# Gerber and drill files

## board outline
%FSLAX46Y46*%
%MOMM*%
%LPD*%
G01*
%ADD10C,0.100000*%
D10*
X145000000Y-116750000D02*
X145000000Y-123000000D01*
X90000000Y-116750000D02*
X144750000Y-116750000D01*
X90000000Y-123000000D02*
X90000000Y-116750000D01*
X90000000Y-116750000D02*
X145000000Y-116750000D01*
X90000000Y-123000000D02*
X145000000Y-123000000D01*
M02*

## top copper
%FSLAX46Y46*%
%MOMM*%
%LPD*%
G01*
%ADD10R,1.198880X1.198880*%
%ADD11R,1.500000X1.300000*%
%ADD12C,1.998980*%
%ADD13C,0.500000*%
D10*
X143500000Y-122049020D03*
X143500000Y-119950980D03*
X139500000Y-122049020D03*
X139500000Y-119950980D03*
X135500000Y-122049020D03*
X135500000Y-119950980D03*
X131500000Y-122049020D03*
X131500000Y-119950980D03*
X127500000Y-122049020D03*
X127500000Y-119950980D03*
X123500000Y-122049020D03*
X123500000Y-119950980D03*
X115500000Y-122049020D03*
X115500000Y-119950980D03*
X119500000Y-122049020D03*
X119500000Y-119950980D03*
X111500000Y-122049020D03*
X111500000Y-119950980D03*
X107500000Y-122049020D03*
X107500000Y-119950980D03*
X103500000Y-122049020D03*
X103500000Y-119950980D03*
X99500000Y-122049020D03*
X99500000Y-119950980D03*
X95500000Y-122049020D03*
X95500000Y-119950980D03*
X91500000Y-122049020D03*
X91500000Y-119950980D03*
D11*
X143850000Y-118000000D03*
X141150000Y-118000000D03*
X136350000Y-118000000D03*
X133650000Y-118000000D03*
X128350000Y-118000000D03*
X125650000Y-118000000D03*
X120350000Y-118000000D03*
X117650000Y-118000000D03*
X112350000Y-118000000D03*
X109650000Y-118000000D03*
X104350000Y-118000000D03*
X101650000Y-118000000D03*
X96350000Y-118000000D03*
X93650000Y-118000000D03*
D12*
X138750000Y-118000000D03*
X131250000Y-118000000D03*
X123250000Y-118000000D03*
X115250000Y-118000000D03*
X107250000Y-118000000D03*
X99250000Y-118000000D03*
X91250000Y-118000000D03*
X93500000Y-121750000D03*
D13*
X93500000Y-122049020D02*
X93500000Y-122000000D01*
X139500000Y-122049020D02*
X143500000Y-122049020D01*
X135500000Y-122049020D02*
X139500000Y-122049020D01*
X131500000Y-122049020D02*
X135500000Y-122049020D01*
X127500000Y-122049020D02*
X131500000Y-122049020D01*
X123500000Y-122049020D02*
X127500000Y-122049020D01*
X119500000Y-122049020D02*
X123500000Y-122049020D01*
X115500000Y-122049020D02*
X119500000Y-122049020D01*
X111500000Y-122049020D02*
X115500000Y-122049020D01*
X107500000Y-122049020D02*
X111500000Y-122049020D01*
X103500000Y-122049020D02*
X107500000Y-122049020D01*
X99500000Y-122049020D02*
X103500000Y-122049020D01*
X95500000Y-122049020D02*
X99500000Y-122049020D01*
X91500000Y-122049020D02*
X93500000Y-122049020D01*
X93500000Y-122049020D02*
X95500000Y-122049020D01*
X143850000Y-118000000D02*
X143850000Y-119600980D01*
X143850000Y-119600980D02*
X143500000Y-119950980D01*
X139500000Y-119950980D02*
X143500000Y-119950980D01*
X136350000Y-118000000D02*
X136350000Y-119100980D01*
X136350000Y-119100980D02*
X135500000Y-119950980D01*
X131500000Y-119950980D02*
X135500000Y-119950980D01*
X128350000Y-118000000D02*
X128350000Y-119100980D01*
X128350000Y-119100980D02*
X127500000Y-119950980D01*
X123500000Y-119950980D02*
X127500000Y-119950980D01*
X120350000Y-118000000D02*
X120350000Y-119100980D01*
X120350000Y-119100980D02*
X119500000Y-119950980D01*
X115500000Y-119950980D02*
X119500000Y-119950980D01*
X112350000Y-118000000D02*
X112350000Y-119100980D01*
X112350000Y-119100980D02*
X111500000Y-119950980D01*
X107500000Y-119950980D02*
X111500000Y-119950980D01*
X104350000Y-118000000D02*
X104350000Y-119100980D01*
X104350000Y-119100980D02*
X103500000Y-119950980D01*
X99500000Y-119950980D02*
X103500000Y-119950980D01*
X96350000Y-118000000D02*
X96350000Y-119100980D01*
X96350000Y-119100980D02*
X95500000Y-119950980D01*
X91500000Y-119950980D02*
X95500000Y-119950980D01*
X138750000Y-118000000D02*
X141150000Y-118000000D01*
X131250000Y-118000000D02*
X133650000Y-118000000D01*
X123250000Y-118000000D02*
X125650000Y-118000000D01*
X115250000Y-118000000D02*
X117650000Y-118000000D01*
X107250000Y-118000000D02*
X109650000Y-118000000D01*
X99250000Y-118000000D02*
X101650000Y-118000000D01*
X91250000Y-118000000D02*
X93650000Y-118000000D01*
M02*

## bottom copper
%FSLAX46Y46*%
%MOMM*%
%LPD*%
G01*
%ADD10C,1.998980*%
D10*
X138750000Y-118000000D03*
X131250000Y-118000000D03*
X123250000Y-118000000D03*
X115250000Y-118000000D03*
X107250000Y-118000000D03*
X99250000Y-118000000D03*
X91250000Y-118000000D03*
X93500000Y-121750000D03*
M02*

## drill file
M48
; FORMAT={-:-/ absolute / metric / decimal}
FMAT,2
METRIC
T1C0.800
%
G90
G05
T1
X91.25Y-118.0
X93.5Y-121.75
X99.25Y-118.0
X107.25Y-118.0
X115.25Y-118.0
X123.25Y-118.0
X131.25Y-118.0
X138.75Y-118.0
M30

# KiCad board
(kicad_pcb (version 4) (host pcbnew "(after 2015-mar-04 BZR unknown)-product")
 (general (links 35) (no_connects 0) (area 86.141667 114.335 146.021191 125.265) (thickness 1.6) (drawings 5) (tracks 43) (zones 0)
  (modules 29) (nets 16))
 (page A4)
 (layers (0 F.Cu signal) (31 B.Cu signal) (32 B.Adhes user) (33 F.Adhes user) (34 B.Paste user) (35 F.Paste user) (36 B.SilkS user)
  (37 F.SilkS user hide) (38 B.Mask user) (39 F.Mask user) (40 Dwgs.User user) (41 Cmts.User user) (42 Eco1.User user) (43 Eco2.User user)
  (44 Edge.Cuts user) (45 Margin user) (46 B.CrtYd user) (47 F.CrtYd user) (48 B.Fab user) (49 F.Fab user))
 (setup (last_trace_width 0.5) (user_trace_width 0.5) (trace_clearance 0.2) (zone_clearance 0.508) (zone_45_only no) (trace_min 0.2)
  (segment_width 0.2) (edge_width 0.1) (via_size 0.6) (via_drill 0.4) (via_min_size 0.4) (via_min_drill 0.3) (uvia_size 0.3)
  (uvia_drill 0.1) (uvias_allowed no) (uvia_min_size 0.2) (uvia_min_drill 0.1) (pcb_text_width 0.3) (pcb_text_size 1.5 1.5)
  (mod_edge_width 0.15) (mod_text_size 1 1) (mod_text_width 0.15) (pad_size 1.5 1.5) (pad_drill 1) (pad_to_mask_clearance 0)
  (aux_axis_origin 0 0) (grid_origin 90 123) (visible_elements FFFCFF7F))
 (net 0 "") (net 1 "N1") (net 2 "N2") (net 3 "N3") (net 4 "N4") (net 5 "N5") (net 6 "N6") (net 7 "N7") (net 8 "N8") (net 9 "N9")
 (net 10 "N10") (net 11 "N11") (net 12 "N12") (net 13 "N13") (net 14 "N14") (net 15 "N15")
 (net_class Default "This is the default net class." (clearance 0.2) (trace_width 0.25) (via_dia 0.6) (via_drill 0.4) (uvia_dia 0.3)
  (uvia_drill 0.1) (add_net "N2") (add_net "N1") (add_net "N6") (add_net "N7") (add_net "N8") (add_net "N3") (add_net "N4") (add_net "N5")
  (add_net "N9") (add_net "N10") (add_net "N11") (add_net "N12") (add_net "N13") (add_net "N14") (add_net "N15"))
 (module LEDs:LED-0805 (layer F.Cu) (at 143.5 121 270)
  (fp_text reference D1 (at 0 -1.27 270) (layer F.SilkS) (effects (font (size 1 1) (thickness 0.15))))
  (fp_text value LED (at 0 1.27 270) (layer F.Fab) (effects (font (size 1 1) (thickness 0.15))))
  (pad 2 smd rect (at 1.04902 0 90) (size 1.19888 1.19888) (layers F.Cu F.Paste F.Mask) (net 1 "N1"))
  (pad 1 smd rect (at -1.04902 0 90) (size 1.19888 1.19888) (layers F.Cu F.Paste F.Mask) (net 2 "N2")))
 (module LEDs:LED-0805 (layer F.Cu) (at 139.5 121 270)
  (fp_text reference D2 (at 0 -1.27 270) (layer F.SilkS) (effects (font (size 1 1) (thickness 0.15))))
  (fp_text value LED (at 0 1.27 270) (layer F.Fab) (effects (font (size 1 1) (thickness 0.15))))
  (pad 2 smd rect (at 1.04902 0 90) (size 1.19888 1.19888) (layers F.Cu F.Paste F.Mask) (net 1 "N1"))
  (pad 1 smd rect (at -1.04902 0 90) (size 1.19888 1.19888) (layers F.Cu F.Paste F.Mask) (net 2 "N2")))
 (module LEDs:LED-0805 (layer F.Cu) (at 135.5 121 270)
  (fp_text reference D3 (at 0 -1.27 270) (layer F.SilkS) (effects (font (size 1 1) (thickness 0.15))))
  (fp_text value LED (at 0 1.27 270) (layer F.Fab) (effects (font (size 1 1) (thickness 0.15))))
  (pad 2 smd rect (at 1.04902 0 90) (size 1.19888 1.19888) (layers F.Cu F.Paste F.Mask) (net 1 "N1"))
  (pad 1 smd rect (at -1.04902 0 90) (size 1.19888 1.19888) (layers F.Cu F.Paste F.Mask) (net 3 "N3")))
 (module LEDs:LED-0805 (layer F.Cu) (at 131.5 121 270)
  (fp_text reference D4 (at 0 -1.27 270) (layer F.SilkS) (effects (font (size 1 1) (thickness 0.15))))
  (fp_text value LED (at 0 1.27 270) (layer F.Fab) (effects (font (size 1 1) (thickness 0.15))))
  (pad 2 smd rect (at 1.04902 0 90) (size 1.19888 1.19888) (layers F.Cu F.Paste F.Mask) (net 1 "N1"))
  (pad 1 smd rect (at -1.04902 0 90) (size 1.19888 1.19888) (layers F.Cu F.Paste F.Mask) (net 3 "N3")))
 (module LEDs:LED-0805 (layer F.Cu) (at 127.5 121 270)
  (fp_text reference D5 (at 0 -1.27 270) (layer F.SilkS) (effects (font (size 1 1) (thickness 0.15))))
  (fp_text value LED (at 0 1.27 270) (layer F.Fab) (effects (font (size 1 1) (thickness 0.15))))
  (pad 2 smd rect (at 1.04902 0 90) (size 1.19888 1.19888) (layers F.Cu F.Paste F.Mask) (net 1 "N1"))
  (pad 1 smd rect (at -1.04902 0 90) (size 1.19888 1.19888) (layers F.Cu F.Paste F.Mask) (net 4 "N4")))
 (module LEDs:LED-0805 (layer F.Cu) (at 123.5 121 270)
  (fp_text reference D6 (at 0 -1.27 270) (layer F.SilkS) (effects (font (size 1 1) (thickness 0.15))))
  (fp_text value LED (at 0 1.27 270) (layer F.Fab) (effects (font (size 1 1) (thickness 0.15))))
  (pad 2 smd rect (at 1.04902 0 90) (size 1.19888 1.19888) (layers F.Cu F.Paste F.Mask) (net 1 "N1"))
  (pad 1 smd rect (at -1.04902 0 90) (size 1.19888 1.19888) (layers F.Cu F.Paste F.Mask) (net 4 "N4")))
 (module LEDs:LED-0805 (layer F.Cu) (at 115.5 121 270)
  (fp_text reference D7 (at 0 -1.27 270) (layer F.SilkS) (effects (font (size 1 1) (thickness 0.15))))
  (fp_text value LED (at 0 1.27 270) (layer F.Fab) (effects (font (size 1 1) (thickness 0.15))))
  (pad 2 smd rect (at 1.04902 0 90) (size 1.19888 1.19888) (layers F.Cu F.Paste F.Mask) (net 1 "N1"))
  (pad 1 smd rect (at -1.04902 0 90) (size 1.19888 1.19888) (layers F.Cu F.Paste F.Mask) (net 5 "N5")))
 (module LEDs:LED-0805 (layer F.Cu) (at 119.5 121 270)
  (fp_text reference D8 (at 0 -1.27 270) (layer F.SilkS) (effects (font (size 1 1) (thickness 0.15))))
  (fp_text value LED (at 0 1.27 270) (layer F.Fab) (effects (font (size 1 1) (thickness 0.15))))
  (pad 2 smd rect (at 1.04902 0 90) (size 1.19888 1.19888) (layers F.Cu F.Paste F.Mask) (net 1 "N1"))
  (pad 1 smd rect (at -1.04902 0 90) (size 1.19888 1.19888) (layers F.Cu F.Paste F.Mask) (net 5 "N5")))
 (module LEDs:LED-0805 (layer F.Cu) (at 111.5 121 270)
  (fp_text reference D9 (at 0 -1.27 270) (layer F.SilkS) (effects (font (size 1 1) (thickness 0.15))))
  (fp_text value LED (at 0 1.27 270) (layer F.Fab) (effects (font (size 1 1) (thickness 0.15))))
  (pad 2 smd rect (at 1.04902 0 90) (size 1.19888 1.19888) (layers F.Cu F.Paste F.Mask) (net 1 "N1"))
  (pad 1 smd rect (at -1.04902 0 90) (size 1.19888 1.19888) (layers F.Cu F.Paste F.Mask) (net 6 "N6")))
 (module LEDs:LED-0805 (layer F.Cu) (at 107.5 121 270)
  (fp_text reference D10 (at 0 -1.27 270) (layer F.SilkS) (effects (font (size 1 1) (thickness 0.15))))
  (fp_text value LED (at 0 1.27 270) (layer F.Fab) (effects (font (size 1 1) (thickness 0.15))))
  (pad 2 smd rect (at 1.04902 0 90) (size 1.19888 1.19888) (layers F.Cu F.Paste F.Mask) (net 1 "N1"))
  (pad 1 smd rect (at -1.04902 0 90) (size 1.19888 1.19888) (layers F.Cu F.Paste F.Mask) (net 6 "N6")))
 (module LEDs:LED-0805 (layer F.Cu) (at 103.5 121 270)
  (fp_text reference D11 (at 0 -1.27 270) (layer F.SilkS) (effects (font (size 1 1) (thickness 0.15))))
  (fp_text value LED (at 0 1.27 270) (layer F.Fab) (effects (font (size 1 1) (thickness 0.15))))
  (pad 2 smd rect (at 1.04902 0 90) (size 1.19888 1.19888) (layers F.Cu F.Paste F.Mask) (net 1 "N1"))
  (pad 1 smd rect (at -1.04902 0 90) (size 1.19888 1.19888) (layers F.Cu F.Paste F.Mask) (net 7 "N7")))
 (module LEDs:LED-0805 (layer F.Cu) (at 99.5 121 270)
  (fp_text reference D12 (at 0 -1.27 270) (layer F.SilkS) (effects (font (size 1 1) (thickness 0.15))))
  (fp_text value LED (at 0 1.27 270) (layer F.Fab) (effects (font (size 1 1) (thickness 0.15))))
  (pad 2 smd rect (at 1.04902 0 90) (size 1.19888 1.19888) (layers F.Cu F.Paste F.Mask) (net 1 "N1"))
  (pad 1 smd rect (at -1.04902 0 90) (size 1.19888 1.19888) (layers F.Cu F.Paste F.Mask) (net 7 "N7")))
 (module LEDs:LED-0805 (layer F.Cu) (at 95.5 121 270)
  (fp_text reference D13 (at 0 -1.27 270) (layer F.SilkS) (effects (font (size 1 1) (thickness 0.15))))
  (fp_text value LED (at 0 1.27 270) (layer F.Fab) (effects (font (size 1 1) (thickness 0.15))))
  (pad 2 smd rect (at 1.04902 0 90) (size 1.19888 1.19888) (layers F.Cu F.Paste F.Mask) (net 1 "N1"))
  (pad 1 smd rect (at -1.04902 0 90) (size 1.19888 1.19888) (layers F.Cu F.Paste F.Mask) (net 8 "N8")))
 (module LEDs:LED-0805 (layer F.Cu) (at 91.5 121 270)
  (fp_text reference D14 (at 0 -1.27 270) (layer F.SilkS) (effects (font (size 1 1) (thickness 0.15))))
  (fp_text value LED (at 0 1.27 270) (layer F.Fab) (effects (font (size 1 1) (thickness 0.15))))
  (pad 2 smd rect (at 1.04902 0 90) (size 1.19888 1.19888) (layers F.Cu F.Paste F.Mask) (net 1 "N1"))
  (pad 1 smd rect (at -1.04902 0 90) (size 1.19888 1.19888) (layers F.Cu F.Paste F.Mask) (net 8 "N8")))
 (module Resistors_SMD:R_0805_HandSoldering (layer F.Cu) (at 142.5 118 180)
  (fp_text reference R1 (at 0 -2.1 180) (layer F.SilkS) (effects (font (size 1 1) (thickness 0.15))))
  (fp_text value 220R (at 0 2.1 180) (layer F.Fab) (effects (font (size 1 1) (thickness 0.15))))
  (pad 1 smd rect (at -1.35 0 180) (size 1.5 1.3) (layers F.Cu F.Paste F.Mask) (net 2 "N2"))
  (pad 2 smd rect (at 1.35 0 180) (size 1.5 1.3) (layers F.Cu F.Paste F.Mask) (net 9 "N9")))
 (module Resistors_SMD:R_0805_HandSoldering (layer F.Cu) (at 135 118 180)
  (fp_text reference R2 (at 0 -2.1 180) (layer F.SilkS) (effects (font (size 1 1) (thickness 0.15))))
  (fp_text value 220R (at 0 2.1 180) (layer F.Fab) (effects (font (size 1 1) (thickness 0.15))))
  (pad 1 smd rect (at -1.35 0 180) (size 1.5 1.3) (layers F.Cu F.Paste F.Mask) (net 3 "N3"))
  (pad 2 smd rect (at 1.35 0 180) (size 1.5 1.3) (layers F.Cu F.Paste F.Mask) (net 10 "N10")))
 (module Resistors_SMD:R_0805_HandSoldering (layer F.Cu) (at 127 118 180)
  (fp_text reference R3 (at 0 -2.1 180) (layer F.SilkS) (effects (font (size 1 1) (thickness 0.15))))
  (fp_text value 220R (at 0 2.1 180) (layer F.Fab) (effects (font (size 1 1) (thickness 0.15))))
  (pad 1 smd rect (at -1.35 0 180) (size 1.5 1.3) (layers F.Cu F.Paste F.Mask) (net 4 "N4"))
  (pad 2 smd rect (at 1.35 0 180) (size 1.5 1.3) (layers F.Cu F.Paste F.Mask) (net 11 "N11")))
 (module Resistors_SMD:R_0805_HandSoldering (layer F.Cu) (at 119 118 180)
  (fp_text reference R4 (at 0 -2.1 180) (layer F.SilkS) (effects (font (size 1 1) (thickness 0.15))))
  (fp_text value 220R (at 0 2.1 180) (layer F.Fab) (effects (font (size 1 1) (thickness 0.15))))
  (pad 1 smd rect (at -1.35 0 180) (size 1.5 1.3) (layers F.Cu F.Paste F.Mask) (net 5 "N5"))
  (pad 2 smd rect (at 1.35 0 180) (size 1.5 1.3) (layers F.Cu F.Paste F.Mask) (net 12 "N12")))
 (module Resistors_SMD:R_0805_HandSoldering (layer F.Cu) (at 111 118 180)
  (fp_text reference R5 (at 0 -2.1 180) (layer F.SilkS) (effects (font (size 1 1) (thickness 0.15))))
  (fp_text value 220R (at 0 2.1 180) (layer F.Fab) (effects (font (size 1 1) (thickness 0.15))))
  (pad 1 smd rect (at -1.35 0 180) (size 1.5 1.3) (layers F.Cu F.Paste F.Mask) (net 6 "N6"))
  (pad 2 smd rect (at 1.35 0 180) (size 1.5 1.3) (layers F.Cu F.Paste F.Mask) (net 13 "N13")))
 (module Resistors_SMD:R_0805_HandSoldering (layer F.Cu) (at 103 118 180)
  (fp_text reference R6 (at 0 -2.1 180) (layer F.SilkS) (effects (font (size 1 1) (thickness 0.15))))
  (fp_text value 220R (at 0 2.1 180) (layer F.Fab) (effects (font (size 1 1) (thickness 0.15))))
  (pad 1 smd rect (at -1.35 0 180) (size 1.5 1.3) (layers F.Cu F.Paste F.Mask) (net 7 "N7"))
  (pad 2 smd rect (at 1.35 0 180) (size 1.5 1.3) (layers F.Cu F.Paste F.Mask) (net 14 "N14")))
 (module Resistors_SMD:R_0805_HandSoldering (layer F.Cu) (at 95 118 180)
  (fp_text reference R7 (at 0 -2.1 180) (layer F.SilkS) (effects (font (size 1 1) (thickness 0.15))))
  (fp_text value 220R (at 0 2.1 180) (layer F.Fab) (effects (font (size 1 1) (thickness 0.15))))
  (pad 1 smd rect (at -1.35 0 180) (size 1.5 1.3) (layers F.Cu F.Paste F.Mask) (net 8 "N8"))
  (pad 2 smd rect (at 1.35 0 180) (size 1.5 1.3) (layers F.Cu F.Paste F.Mask) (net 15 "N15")))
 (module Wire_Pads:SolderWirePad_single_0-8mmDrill (layer B.Cu) (at 138.75 118)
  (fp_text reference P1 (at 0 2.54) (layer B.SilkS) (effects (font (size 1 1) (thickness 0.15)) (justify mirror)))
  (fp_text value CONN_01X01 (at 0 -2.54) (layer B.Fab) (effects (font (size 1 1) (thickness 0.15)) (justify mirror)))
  (pad 1 thru_hole circle (at 0 0) (size 1.99898 1.99898) (drill 0.8001) (layers *.Cu *.Mask B.SilkS) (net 9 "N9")))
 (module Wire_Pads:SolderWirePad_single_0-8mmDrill (layer B.Cu) (at 131.25 118)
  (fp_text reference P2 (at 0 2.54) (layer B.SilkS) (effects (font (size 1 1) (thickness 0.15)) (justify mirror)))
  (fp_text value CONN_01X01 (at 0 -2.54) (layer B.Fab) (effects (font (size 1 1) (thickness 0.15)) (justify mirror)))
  (pad 1 thru_hole circle (at 0 0) (size 1.99898 1.99898) (drill 0.8001) (layers *.Cu *.Mask B.SilkS) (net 10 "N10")))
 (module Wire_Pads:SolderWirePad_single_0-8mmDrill (layer B.Cu) (at 123.25 118)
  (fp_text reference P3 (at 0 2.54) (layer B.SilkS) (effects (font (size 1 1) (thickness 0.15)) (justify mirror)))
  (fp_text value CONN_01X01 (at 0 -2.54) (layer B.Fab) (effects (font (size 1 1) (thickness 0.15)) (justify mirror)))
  (pad 1 thru_hole circle (at 0 0) (size 1.99898 1.99898) (drill 0.8001) (layers *.Cu *.Mask B.SilkS) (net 11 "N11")))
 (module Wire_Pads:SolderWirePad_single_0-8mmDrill (layer B.Cu) (at 115.25 118)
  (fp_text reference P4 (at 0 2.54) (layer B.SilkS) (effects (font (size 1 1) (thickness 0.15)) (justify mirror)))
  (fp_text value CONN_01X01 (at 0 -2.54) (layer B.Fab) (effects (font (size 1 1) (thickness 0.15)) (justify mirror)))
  (pad 1 thru_hole circle (at 0 0) (size 1.99898 1.99898) (drill 0.8001) (layers *.Cu *.Mask B.SilkS) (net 12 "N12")))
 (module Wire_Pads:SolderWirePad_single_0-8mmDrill (layer B.Cu) (at 107.25 118)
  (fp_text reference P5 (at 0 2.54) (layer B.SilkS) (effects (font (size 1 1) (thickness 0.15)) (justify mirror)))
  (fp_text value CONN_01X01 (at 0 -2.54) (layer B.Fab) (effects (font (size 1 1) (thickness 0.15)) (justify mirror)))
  (pad 1 thru_hole circle (at 0 0) (size 1.99898 1.99898) (drill 0.8001) (layers *.Cu *.Mask B.SilkS) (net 13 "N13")))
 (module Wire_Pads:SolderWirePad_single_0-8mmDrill (layer B.Cu) (at 99.25 118)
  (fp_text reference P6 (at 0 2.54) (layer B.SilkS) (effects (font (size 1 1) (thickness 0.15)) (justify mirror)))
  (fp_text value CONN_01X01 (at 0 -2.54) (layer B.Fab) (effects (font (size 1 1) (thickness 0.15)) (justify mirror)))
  (pad 1 thru_hole circle (at 0 0) (size 1.99898 1.99898) (drill 0.8001) (layers *.Cu *.Mask B.SilkS) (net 14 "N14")))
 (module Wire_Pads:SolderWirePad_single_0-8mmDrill (layer B.Cu) (at 91.25 118)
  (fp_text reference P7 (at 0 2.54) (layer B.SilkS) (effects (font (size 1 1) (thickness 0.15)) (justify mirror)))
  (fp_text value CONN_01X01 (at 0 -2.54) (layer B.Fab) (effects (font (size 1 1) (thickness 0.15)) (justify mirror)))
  (pad 1 thru_hole circle (at 0 0) (size 1.99898 1.99898) (drill 0.8001) (layers *.Cu *.Mask B.SilkS) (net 15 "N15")))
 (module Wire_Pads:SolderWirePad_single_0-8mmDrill (layer B.Cu) (at 93.5 121.75)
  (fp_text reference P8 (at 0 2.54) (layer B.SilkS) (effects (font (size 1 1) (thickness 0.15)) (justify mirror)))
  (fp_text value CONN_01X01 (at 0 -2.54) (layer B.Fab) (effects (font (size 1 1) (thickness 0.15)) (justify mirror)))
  (pad 1 thru_hole circle (at 0 0) (size 1.99898 1.99898) (drill 0.8001) (layers *.Cu *.Mask B.SilkS) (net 1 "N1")))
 (gr_line (start 145 116.75) (end 145 123) (angle 90) (layer Edge.Cuts) (width 0.1))
 (gr_line (start 90 116.75) (end 144.75 116.75) (angle 90) (layer Edge.Cuts) (width 0.1))
 (gr_line (start 90 123) (end 90 116.75) (angle 90) (layer Edge.Cuts) (width 0.1))
 (gr_line (start 90 116.75) (end 145 116.75) (angle 90) (layer Edge.Cuts) (width 0.1))
 (gr_line (start 90 123) (end 145 123) (angle 90) (layer Edge.Cuts) (width 0.1))
 (segment (start 93.5 122.04902) (end 93.5 122) (width 0.5) (layer F.Cu) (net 1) (status 20))
 (segment (start 139.5 122.04902) (end 143.5 122.04902) (width 0.5) (layer F.Cu) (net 1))
 (segment (start 135.5 122.04902) (end 139.5 122.04902) (width 0.5) (layer F.Cu) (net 1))
 (segment (start 131.5 122.04902) (end 135.5 122.04902) (width 0.5) (layer F.Cu) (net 1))
 (segment (start 127.5 122.04902) (end 131.5 122.04902) (width 0.5) (layer F.Cu) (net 1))
 (segment (start 123.5 122.04902) (end 127.5 122.04902) (width 0.5) (layer F.Cu) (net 1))
 (segment (start 119.5 122.04902) (end 123.5 122.04902) (width 0.5) (layer F.Cu) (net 1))
 (segment (start 115.5 122.04902) (end 119.5 122.04902) (width 0.5) (layer F.Cu) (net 1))
 (segment (start 111.5 122.04902) (end 115.5 122.04902) (width 0.5) (layer F.Cu) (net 1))
 (segment (start 107.5 122.04902) (end 111.5 122.04902) (width 0.5) (layer F.Cu) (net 1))
 (segment (start 103.5 122.04902) (end 107.5 122.04902) (width 0.5) (layer F.Cu) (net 1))
 (segment (start 99.5 122.04902) (end 103.5 122.04902) (width 0.5) (layer F.Cu) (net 1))
 (segment (start 95.5 122.04902) (end 99.5 122.04902) (width 0.5) (layer F.Cu) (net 1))
 (segment (start 91.5 122.04902) (end 93.5 122.04902) (width 0.5) (layer F.Cu) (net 1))
 (segment (start 93.5 122.04902) (end 95.5 122.04902) (width 0.5) (layer F.Cu) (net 1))
 (segment (start 143.85 118) (end 143.85 119.60098) (width 0.5) (layer F.Cu) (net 2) (status C00000))
 (segment (start 143.85 119.60098) (end 143.5 119.95098) (width 0.5) (layer F.Cu) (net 2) (status C00000))
 (segment (start 139.5 119.95098) (end 143.5 119.95098) (width 0.5) (layer F.Cu) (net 2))
 (segment (start 136.35 118) (end 136.35 119.10098) (width 0.5) (layer F.Cu) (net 3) (status 400000))
 (segment (start 136.35 119.10098) (end 135.5 119.95098) (width 0.5) (layer F.Cu) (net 3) (status 800000))
 (segment (start 131.5 119.95098) (end 135.5 119.95098) (width 0.5) (layer F.Cu) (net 3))
 (segment (start 128.35 118) (end 128.35 119.10098) (width 0.5) (layer F.Cu) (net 4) (status 400000))
 (segment (start 128.35 119.10098) (end 127.5 119.95098) (width 0.5) (layer F.Cu) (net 4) (status 800000))
 (segment (start 123.5 119.95098) (end 127.5 119.95098) (width 0.5) (layer F.Cu) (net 4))
 (segment (start 120.35 118) (end 120.35 119.10098) (width 0.5) (layer F.Cu) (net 5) (status 400000))
 (segment (start 120.35 119.10098) (end 119.5 119.95098) (width 0.5) (layer F.Cu) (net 5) (status 800000))
 (segment (start 115.5 119.95098) (end 119.5 119.95098) (width 0.5) (layer F.Cu) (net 5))
 (segment (start 112.35 118) (end 112.35 119.10098) (width 0.5) (layer F.Cu) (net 6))
 (segment (start 112.35 119.10098) (end 111.5 119.95098) (width 0.5) (layer F.Cu) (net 6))
 (segment (start 107.5 119.95098) (end 111.5 119.95098) (width 0.5) (layer F.Cu) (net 6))
 (segment (start 104.35 118) (end 104.35 119.10098) (width 0.5) (layer F.Cu) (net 7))
 (segment (start 104.35 119.10098) (end 103.5 119.95098) (width 0.5) (layer F.Cu) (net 7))
 (segment (start 99.5 119.95098) (end 103.5 119.95098) (width 0.5) (layer F.Cu) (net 7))
 (segment (start 96.35 118) (end 96.35 119.10098) (width 0.5) (layer F.Cu) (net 8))
 (segment (start 96.35 119.10098) (end 95.5 119.95098) (width 0.5) (layer F.Cu) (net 8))
 (segment (start 91.5 119.95098) (end 95.5 119.95098) (width 0.5) (layer F.Cu) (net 8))
 (segment (start 138.75 118) (end 141.15 118) (width 0.5) (layer F.Cu) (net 9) (status C00000))
 (segment (start 131.25 118) (end 133.65 118) (width 0.5) (layer F.Cu) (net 10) (status C00000))
 (segment (start 123.25 118) (end 125.65 118) (width 0.5) (layer F.Cu) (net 11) (status C00000))
 (segment (start 115.25 118) (end 117.65 118) (width 0.5) (layer F.Cu) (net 12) (status C00000))
 (segment (start 107.25 118) (end 109.65 118) (width 0.5) (layer F.Cu) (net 13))
 (segment (start 99.25 118) (end 101.65 118) (width 0.5) (layer F.Cu) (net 14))
 (segment (start 91.25 118) (end 93.65 118) (width 0.5) (layer F.Cu) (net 15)))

